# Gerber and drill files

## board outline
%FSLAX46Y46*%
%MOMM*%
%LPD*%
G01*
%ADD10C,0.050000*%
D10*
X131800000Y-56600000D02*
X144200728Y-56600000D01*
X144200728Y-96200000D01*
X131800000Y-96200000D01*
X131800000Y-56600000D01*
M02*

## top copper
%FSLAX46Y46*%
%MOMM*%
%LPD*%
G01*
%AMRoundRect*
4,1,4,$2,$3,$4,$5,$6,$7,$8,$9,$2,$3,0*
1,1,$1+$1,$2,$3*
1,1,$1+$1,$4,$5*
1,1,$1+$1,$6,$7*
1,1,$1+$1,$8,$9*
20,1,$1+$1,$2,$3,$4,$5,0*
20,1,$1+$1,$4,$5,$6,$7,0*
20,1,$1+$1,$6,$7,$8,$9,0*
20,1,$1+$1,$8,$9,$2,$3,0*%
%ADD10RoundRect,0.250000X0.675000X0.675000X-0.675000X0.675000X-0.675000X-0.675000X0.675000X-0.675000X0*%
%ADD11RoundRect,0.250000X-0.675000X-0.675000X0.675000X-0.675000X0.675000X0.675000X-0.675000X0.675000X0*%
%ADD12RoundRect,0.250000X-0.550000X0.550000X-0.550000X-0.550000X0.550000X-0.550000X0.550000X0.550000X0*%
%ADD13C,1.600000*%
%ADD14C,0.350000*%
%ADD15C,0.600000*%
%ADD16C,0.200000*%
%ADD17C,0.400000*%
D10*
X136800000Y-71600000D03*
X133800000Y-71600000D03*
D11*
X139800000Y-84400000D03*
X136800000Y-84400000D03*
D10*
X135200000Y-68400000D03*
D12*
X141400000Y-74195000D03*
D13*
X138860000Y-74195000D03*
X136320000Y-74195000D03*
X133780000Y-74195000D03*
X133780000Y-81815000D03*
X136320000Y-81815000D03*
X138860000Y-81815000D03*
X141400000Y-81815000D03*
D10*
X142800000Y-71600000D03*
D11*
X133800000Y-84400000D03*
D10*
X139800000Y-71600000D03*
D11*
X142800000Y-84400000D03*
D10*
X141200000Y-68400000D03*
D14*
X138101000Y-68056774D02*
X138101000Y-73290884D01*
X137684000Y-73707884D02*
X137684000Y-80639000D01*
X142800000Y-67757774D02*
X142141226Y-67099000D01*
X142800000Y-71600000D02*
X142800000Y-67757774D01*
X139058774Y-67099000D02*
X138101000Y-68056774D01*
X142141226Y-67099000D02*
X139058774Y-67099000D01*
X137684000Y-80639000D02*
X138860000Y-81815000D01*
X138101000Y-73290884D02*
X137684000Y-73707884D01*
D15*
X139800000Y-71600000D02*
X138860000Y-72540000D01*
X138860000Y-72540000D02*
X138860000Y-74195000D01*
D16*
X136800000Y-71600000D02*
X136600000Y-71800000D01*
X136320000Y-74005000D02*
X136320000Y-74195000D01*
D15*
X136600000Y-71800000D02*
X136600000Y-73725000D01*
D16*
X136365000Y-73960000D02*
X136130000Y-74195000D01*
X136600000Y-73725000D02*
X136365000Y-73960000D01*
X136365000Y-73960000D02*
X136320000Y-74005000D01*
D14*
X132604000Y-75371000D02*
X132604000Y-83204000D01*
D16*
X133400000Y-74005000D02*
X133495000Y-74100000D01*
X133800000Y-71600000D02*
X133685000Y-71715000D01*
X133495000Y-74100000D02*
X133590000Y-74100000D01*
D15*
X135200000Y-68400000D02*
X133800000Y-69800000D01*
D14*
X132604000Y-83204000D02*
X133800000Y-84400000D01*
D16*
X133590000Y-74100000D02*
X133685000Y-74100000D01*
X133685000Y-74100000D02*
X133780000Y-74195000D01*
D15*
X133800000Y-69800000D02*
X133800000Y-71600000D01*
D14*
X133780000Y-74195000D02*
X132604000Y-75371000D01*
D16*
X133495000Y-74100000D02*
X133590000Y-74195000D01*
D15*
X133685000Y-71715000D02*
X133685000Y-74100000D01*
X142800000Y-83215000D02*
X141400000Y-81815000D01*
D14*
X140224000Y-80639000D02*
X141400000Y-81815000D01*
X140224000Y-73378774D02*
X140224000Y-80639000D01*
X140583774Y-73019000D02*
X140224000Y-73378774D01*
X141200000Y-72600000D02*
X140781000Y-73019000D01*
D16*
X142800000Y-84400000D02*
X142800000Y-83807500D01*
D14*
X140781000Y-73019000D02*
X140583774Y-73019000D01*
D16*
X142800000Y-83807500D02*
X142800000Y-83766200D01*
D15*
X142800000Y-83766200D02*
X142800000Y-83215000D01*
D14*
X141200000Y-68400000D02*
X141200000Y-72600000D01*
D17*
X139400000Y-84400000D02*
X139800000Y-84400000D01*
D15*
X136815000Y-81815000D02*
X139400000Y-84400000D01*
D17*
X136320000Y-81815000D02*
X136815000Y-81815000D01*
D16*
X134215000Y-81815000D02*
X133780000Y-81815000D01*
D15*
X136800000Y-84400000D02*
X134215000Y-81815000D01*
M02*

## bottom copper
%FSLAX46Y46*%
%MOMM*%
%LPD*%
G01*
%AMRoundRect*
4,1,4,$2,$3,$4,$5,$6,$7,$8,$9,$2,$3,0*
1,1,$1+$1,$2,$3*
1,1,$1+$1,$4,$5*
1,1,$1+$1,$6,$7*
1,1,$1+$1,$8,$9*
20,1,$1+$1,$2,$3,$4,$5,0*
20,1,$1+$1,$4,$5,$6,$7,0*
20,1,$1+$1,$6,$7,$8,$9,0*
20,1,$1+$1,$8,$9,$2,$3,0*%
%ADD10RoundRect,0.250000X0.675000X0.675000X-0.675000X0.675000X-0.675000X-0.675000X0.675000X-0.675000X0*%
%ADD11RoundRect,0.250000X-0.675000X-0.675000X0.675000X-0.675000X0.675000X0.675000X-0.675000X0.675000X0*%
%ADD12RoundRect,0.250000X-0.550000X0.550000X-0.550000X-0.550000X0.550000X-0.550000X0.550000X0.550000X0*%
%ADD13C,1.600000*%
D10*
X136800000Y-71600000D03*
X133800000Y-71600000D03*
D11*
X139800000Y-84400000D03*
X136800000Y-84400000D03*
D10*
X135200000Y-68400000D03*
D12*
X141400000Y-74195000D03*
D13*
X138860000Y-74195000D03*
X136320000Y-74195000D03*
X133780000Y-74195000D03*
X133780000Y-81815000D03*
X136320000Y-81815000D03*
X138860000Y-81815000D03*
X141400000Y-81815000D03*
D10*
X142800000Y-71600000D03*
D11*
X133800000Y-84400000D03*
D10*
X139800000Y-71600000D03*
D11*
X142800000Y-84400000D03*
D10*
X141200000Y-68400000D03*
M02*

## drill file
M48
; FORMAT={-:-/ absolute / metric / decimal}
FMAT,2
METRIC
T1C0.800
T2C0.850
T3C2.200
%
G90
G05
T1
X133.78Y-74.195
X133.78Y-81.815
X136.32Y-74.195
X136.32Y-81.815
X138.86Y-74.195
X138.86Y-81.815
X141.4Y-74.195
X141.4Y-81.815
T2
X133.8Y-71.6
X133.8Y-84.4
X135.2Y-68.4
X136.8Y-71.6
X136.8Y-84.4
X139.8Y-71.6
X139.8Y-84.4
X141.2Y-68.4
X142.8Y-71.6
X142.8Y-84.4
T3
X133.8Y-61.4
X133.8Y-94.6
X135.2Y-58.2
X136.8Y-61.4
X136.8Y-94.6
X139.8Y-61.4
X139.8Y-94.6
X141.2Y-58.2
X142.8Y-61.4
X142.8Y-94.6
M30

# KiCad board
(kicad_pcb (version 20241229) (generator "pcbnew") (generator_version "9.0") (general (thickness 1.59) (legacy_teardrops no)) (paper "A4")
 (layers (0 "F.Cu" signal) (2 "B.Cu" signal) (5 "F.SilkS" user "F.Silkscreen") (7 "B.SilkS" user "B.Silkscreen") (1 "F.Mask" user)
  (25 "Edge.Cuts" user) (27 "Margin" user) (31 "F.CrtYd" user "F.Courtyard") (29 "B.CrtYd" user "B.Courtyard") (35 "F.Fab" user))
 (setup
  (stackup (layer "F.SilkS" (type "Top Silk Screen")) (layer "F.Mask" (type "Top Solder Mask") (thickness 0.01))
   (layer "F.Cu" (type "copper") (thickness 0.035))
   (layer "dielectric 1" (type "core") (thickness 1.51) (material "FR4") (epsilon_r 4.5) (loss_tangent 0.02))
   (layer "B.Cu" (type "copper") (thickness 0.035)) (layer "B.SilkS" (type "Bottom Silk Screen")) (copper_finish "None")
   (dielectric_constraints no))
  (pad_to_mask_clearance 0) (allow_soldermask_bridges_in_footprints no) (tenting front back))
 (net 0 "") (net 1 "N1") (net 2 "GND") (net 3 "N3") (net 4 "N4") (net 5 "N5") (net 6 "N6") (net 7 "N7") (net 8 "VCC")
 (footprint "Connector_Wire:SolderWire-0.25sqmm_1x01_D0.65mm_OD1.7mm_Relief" (layer "F.Cu") (at 136.8 71.6 180)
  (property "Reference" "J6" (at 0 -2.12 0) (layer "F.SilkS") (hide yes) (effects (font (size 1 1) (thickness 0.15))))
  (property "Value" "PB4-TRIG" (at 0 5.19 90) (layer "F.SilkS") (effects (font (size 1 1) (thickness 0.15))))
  (pad "" np_thru_hole circle (at 0 10.2 180) (size 2.2 2.2) (drill 2.2) (layers "*.Cu" "*.Mask"))
  (pad "1" thru_hole roundrect (at 0 0 180) (size 1.85 1.85) (drill 0.85) (layers "*.Cu" "*.Mask") (remove_unused_layers no)
   (roundrect_rratio 0.135135) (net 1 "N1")))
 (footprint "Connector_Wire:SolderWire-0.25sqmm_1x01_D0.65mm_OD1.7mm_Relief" (layer "F.Cu") (at 133.8 71.6 180)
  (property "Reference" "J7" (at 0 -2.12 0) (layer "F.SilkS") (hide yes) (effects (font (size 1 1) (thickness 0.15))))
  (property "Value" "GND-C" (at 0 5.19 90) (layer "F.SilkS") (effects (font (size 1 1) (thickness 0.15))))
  (pad "" np_thru_hole circle (at 0 10.2 180) (size 2.2 2.2) (drill 2.2) (layers "*.Cu" "*.Mask"))
  (pad "1" thru_hole roundrect (at 0 0 180) (size 1.85 1.85) (drill 0.85) (layers "*.Cu" "*.Mask") (remove_unused_layers no)
   (roundrect_rratio 0.135135) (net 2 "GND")))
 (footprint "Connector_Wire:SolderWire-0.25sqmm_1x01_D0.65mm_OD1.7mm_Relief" (layer "F.Cu") (at 139.8 84.4)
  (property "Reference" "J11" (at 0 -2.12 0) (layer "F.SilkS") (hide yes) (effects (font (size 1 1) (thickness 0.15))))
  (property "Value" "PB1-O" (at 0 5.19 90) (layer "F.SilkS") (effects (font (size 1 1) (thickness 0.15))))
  (pad "" np_thru_hole circle (at 0 10.2) (size 2.2 2.2) (drill 2.2) (layers "*.Cu" "*.Mask"))
  (pad "1" thru_hole roundrect (at 0 0) (size 1.85 1.85) (drill 0.85) (layers "*.Cu" "*.Mask") (remove_unused_layers no)
   (roundrect_rratio 0.135135) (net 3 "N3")))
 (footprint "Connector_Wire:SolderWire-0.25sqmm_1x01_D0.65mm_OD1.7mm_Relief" (layer "F.Cu") (at 136.8 84.4)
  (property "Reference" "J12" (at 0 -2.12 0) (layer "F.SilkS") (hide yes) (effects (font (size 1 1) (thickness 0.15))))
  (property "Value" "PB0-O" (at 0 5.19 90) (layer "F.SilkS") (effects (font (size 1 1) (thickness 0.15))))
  (pad "" np_thru_hole circle (at 0 10.2) (size 2.2 2.2) (drill 2.2) (layers "*.Cu" "*.Mask"))
  (pad "1" thru_hole roundrect (at 0 0) (size 1.85 1.85) (drill 0.85) (layers "*.Cu" "*.Mask") (remove_unused_layers no)
   (roundrect_rratio 0.135135) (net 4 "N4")))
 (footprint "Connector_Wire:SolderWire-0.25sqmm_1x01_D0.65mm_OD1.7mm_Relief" (layer "F.Cu") (at 135.2 68.4 180)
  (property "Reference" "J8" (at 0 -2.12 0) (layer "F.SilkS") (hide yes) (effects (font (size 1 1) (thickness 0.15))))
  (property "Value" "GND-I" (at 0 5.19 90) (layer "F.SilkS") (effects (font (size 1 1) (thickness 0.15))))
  (pad "" np_thru_hole circle (at 0 10.2 180) (size 2.2 2.2) (drill 2.2) (layers "*.Cu" "*.Mask"))
  (pad "1" thru_hole roundrect (at 0 0 180) (size 1.85 1.85) (drill 0.85) (layers "*.Cu" "*.Mask") (remove_unused_layers no)
   (roundrect_rratio 0.135135) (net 2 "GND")))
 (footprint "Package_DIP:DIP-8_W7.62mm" (layer "F.Cu") (at 141.4 74.195 -90)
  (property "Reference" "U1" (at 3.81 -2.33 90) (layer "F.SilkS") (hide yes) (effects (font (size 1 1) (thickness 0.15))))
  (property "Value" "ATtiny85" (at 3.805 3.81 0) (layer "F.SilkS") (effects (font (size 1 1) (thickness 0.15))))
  (pad "1" thru_hole roundrect (at 0 0 270) (size 1.6 1.6) (drill 0.8) (layers "*.Cu" "*.Mask") (remove_unused_layers no)
   (roundrect_rratio 0.15625) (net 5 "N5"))
  (pad "2" thru_hole circle (at 0 2.54 270) (size 1.6 1.6) (drill 0.8) (layers "*.Cu" "*.Mask") (remove_unused_layers no) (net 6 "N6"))
  (pad "3" thru_hole circle (at 0 5.08 270) (size 1.6 1.6) (drill 0.8) (layers "*.Cu" "*.Mask") (remove_unused_layers no) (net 1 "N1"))
  (pad "4" thru_hole circle (at 0 7.62 270) (size 1.6 1.6) (drill 0.8) (layers "*.Cu" "*.Mask") (remove_unused_layers no) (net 2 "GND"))
  (pad "5" thru_hole circle (at 7.62 7.62 270) (size 1.6 1.6) (drill 0.8) (layers "*.Cu" "*.Mask") (remove_unused_layers no) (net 4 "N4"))
  (pad "6" thru_hole circle (at 7.62 5.08 270) (size 1.6 1.6) (drill 0.8) (layers "*.Cu" "*.Mask") (remove_unused_layers no) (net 3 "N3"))
  (pad "7" thru_hole circle (at 7.62 2.54 270) (size 1.6 1.6) (drill 0.8) (layers "*.Cu" "*.Mask") (remove_unused_layers no) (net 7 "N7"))
  (pad "8" thru_hole circle (at 7.62 0 270) (size 1.6 1.6) (drill 0.8) (layers "*.Cu" "*.Mask") (remove_unused_layers no) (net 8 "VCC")))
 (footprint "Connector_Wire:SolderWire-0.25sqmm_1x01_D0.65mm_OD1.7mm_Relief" (layer "F.Cu") (at 142.8 71.6 180)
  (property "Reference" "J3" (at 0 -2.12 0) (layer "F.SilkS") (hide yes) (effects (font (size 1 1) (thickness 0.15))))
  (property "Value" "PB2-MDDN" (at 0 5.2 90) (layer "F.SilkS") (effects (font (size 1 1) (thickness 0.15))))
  (pad "" np_thru_hole circle (at 0 10.2 180) (size 2.2 2.2) (drill 2.2) (layers "*.Cu" "*.Mask"))
  (pad "1" thru_hole roundrect (at 0 0 180) (size 1.85 1.85) (drill 0.85) (layers "*.Cu" "*.Mask") (remove_unused_layers no)
   (roundrect_rratio 0.135135) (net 7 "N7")))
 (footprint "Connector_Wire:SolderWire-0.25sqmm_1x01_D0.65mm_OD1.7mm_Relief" (layer "F.Cu") (at 133.8 84.4)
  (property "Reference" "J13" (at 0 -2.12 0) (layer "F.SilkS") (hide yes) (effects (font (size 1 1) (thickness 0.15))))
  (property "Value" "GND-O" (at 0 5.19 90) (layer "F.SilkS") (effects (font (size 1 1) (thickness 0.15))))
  (pad "" np_thru_hole circle (at 0 10.2) (size 2.2 2.2) (drill 2.2) (layers "*.Cu" "*.Mask"))
  (pad "1" thru_hole roundrect (at 0 0) (size 1.85 1.85) (drill 0.85) (layers "*.Cu" "*.Mask") (remove_unused_layers no)
   (roundrect_rratio 0.135135) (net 2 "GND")))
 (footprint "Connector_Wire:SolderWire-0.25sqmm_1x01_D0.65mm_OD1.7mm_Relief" (layer "F.Cu") (at 139.8 71.6 180)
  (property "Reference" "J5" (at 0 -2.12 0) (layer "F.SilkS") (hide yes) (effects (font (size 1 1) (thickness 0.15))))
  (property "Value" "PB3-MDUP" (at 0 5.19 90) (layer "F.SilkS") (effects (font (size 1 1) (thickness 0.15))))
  (pad "" np_thru_hole circle (at 0 10.2 180) (size 2.2 2.2) (drill 2.2) (layers "*.Cu" "*.Mask"))
  (pad "1" thru_hole roundrect (at 0 0 180) (size 1.85 1.85) (drill 0.85) (layers "*.Cu" "*.Mask") (remove_unused_layers no)
   (roundrect_rratio 0.135135) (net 6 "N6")))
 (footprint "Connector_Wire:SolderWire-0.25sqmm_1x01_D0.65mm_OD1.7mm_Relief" (layer "F.Cu") (at 142.8 84.4)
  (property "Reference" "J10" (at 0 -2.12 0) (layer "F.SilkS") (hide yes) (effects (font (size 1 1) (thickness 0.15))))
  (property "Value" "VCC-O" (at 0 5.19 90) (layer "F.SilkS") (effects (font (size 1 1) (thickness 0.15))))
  (pad "" np_thru_hole circle (at 0 10.2) (size 2.2 2.2) (drill 2.2) (layers "*.Cu" "*.Mask"))
  (pad "1" thru_hole roundrect (at 0 0) (size 1.85 1.85) (drill 0.85) (layers "*.Cu" "*.Mask") (remove_unused_layers no)
   (roundrect_rratio 0.135135) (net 8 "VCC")))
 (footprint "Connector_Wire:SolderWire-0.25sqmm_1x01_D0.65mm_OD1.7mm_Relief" (layer "F.Cu") (at 141.2 68.4 180)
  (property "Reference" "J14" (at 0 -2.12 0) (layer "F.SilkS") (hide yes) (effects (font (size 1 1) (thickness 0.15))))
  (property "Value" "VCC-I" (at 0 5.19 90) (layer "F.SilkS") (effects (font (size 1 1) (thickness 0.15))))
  (pad "" np_thru_hole circle (at 0 10.2 180) (size 2.2 2.2) (drill 2.2) (layers "*.Cu" "*.Mask"))
  (pad "1" thru_hole roundrect (at 0 0 180) (size 1.85 1.85) (drill 0.85) (layers "*.Cu" "*.Mask") (remove_unused_layers no)
   (roundrect_rratio 0.135135) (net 8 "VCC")))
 (gr_rect (start 131.8 56.6) (end 144.200728 96.2) (stroke (width 0.05) (type default)) (fill no) (layer "Edge.Cuts"))
 (segment (start 138.101 68.056774) (end 138.101 73.290884) (width 0.35) (layer "F.Cu") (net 7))
 (segment (start 137.684 73.707884) (end 137.684 80.639) (width 0.35) (layer "F.Cu") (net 7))
 (segment (start 142.8 67.757774) (end 142.141226 67.099) (width 0.35) (layer "F.Cu") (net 7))
 (segment (start 142.8 71.6) (end 142.8 67.757774) (width 0.35) (layer "F.Cu") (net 7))
 (segment (start 139.058774 67.099) (end 138.101 68.056774) (width 0.35) (layer "F.Cu") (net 7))
 (segment (start 142.141226 67.099) (end 139.058774 67.099) (width 0.35) (layer "F.Cu") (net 7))
 (segment (start 137.684 80.639) (end 138.86 81.815) (width 0.35) (layer "F.Cu") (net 7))
 (segment (start 138.101 73.290884) (end 137.684 73.707884) (width 0.35) (layer "F.Cu") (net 7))
 (segment (start 139.8 71.6) (end 138.86 72.54) (width 0.6) (layer "F.Cu") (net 6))
 (segment (start 138.86 72.54) (end 138.86 74.195) (width 0.6) (layer "F.Cu") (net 6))
 (segment (start 136.8 71.6) (end 136.6 71.8) (width 0.2) (layer "F.Cu") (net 1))
 (segment (start 136.32 74.005) (end 136.32 74.195) (width 0.2) (layer "F.Cu") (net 1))
 (segment (start 136.6 71.8) (end 136.6 73.725) (width 0.6) (layer "F.Cu") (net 1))
 (segment (start 136.365 73.96) (end 136.13 74.195) (width 0.2) (layer "F.Cu") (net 1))
 (segment (start 136.6 73.725) (end 136.365 73.96) (width 0.2) (layer "F.Cu") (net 1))
 (segment (start 136.365 73.96) (end 136.32 74.005) (width 0.2) (layer "F.Cu") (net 1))
 (segment (start 132.604 75.371) (end 132.604 83.204) (width 0.35) (layer "F.Cu") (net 2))
 (segment (start 133.4 74.005) (end 133.495 74.1) (width 0.2) (layer "F.Cu") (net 2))
 (segment (start 133.8 71.6) (end 133.685 71.715) (width 0.2) (layer "F.Cu") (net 2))
 (segment (start 133.495 74.1) (end 133.59 74.1) (width 0.2) (layer "F.Cu") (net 2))
 (segment (start 135.2 68.4) (end 133.8 69.8) (width 0.6) (layer "F.Cu") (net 2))
 (segment (start 132.604 83.204) (end 133.8 84.4) (width 0.35) (layer "F.Cu") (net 2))
 (segment (start 133.59 74.1) (end 133.685 74.1) (width 0.2) (layer "F.Cu") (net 2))
 (segment (start 133.685 74.1) (end 133.78 74.195) (width 0.2) (layer "F.Cu") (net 2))
 (segment (start 133.8 69.8) (end 133.8 71.6) (width 0.6) (layer "F.Cu") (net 2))
 (segment (start 133.78 74.195) (end 132.604 75.371) (width 0.35) (layer "F.Cu") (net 2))
 (segment (start 133.495 74.1) (end 133.59 74.195) (width 0.2) (layer "F.Cu") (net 2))
 (segment (start 133.685 71.715) (end 133.685 74.1) (width 0.6) (layer "F.Cu") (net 2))
 (segment (start 142.8 83.215) (end 141.4 81.815) (width 0.6) (layer "F.Cu") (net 8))
 (segment (start 140.224 80.639) (end 141.4 81.815) (width 0.35) (layer "F.Cu") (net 8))
 (segment (start 140.224 73.378774) (end 140.224 80.639) (width 0.35) (layer "F.Cu") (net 8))
 (segment (start 140.583774 73.019) (end 140.224 73.378774) (width 0.35) (layer "F.Cu") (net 8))
 (segment (start 141.2 72.6) (end 140.781 73.019) (width 0.35) (layer "F.Cu") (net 8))
 (segment (start 142.8 84.4) (end 142.8 83.8075) (width 0.2) (layer "F.Cu") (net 8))
 (segment (start 140.781 73.019) (end 140.583774 73.019) (width 0.35) (layer "F.Cu") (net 8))
 (segment (start 142.8 83.8075) (end 142.8 83.7662) (width 0.2) (layer "F.Cu") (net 8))
 (segment (start 142.8 83.7662) (end 142.8 83.215) (width 0.6) (layer "F.Cu") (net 8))
 (segment (start 141.2 68.4) (end 141.2 72.6) (width 0.35) (layer "F.Cu") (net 8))
 (segment (start 139.4 84.4) (end 139.8 84.4) (width 0.4) (layer "F.Cu") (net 3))
 (segment (start 136.815 81.815) (end 139.4 84.4) (width 0.6) (layer "F.Cu") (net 3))
 (segment (start 136.32 81.815) (end 136.815 81.815) (width 0.4) (layer "F.Cu") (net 3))
 (segment (start 134.215 81.815) (end 133.78 81.815) (width 0.2) (layer "F.Cu") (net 4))
 (segment (start 136.8 84.4) (end 134.215 81.815) (width 0.6) (layer "F.Cu") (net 4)))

